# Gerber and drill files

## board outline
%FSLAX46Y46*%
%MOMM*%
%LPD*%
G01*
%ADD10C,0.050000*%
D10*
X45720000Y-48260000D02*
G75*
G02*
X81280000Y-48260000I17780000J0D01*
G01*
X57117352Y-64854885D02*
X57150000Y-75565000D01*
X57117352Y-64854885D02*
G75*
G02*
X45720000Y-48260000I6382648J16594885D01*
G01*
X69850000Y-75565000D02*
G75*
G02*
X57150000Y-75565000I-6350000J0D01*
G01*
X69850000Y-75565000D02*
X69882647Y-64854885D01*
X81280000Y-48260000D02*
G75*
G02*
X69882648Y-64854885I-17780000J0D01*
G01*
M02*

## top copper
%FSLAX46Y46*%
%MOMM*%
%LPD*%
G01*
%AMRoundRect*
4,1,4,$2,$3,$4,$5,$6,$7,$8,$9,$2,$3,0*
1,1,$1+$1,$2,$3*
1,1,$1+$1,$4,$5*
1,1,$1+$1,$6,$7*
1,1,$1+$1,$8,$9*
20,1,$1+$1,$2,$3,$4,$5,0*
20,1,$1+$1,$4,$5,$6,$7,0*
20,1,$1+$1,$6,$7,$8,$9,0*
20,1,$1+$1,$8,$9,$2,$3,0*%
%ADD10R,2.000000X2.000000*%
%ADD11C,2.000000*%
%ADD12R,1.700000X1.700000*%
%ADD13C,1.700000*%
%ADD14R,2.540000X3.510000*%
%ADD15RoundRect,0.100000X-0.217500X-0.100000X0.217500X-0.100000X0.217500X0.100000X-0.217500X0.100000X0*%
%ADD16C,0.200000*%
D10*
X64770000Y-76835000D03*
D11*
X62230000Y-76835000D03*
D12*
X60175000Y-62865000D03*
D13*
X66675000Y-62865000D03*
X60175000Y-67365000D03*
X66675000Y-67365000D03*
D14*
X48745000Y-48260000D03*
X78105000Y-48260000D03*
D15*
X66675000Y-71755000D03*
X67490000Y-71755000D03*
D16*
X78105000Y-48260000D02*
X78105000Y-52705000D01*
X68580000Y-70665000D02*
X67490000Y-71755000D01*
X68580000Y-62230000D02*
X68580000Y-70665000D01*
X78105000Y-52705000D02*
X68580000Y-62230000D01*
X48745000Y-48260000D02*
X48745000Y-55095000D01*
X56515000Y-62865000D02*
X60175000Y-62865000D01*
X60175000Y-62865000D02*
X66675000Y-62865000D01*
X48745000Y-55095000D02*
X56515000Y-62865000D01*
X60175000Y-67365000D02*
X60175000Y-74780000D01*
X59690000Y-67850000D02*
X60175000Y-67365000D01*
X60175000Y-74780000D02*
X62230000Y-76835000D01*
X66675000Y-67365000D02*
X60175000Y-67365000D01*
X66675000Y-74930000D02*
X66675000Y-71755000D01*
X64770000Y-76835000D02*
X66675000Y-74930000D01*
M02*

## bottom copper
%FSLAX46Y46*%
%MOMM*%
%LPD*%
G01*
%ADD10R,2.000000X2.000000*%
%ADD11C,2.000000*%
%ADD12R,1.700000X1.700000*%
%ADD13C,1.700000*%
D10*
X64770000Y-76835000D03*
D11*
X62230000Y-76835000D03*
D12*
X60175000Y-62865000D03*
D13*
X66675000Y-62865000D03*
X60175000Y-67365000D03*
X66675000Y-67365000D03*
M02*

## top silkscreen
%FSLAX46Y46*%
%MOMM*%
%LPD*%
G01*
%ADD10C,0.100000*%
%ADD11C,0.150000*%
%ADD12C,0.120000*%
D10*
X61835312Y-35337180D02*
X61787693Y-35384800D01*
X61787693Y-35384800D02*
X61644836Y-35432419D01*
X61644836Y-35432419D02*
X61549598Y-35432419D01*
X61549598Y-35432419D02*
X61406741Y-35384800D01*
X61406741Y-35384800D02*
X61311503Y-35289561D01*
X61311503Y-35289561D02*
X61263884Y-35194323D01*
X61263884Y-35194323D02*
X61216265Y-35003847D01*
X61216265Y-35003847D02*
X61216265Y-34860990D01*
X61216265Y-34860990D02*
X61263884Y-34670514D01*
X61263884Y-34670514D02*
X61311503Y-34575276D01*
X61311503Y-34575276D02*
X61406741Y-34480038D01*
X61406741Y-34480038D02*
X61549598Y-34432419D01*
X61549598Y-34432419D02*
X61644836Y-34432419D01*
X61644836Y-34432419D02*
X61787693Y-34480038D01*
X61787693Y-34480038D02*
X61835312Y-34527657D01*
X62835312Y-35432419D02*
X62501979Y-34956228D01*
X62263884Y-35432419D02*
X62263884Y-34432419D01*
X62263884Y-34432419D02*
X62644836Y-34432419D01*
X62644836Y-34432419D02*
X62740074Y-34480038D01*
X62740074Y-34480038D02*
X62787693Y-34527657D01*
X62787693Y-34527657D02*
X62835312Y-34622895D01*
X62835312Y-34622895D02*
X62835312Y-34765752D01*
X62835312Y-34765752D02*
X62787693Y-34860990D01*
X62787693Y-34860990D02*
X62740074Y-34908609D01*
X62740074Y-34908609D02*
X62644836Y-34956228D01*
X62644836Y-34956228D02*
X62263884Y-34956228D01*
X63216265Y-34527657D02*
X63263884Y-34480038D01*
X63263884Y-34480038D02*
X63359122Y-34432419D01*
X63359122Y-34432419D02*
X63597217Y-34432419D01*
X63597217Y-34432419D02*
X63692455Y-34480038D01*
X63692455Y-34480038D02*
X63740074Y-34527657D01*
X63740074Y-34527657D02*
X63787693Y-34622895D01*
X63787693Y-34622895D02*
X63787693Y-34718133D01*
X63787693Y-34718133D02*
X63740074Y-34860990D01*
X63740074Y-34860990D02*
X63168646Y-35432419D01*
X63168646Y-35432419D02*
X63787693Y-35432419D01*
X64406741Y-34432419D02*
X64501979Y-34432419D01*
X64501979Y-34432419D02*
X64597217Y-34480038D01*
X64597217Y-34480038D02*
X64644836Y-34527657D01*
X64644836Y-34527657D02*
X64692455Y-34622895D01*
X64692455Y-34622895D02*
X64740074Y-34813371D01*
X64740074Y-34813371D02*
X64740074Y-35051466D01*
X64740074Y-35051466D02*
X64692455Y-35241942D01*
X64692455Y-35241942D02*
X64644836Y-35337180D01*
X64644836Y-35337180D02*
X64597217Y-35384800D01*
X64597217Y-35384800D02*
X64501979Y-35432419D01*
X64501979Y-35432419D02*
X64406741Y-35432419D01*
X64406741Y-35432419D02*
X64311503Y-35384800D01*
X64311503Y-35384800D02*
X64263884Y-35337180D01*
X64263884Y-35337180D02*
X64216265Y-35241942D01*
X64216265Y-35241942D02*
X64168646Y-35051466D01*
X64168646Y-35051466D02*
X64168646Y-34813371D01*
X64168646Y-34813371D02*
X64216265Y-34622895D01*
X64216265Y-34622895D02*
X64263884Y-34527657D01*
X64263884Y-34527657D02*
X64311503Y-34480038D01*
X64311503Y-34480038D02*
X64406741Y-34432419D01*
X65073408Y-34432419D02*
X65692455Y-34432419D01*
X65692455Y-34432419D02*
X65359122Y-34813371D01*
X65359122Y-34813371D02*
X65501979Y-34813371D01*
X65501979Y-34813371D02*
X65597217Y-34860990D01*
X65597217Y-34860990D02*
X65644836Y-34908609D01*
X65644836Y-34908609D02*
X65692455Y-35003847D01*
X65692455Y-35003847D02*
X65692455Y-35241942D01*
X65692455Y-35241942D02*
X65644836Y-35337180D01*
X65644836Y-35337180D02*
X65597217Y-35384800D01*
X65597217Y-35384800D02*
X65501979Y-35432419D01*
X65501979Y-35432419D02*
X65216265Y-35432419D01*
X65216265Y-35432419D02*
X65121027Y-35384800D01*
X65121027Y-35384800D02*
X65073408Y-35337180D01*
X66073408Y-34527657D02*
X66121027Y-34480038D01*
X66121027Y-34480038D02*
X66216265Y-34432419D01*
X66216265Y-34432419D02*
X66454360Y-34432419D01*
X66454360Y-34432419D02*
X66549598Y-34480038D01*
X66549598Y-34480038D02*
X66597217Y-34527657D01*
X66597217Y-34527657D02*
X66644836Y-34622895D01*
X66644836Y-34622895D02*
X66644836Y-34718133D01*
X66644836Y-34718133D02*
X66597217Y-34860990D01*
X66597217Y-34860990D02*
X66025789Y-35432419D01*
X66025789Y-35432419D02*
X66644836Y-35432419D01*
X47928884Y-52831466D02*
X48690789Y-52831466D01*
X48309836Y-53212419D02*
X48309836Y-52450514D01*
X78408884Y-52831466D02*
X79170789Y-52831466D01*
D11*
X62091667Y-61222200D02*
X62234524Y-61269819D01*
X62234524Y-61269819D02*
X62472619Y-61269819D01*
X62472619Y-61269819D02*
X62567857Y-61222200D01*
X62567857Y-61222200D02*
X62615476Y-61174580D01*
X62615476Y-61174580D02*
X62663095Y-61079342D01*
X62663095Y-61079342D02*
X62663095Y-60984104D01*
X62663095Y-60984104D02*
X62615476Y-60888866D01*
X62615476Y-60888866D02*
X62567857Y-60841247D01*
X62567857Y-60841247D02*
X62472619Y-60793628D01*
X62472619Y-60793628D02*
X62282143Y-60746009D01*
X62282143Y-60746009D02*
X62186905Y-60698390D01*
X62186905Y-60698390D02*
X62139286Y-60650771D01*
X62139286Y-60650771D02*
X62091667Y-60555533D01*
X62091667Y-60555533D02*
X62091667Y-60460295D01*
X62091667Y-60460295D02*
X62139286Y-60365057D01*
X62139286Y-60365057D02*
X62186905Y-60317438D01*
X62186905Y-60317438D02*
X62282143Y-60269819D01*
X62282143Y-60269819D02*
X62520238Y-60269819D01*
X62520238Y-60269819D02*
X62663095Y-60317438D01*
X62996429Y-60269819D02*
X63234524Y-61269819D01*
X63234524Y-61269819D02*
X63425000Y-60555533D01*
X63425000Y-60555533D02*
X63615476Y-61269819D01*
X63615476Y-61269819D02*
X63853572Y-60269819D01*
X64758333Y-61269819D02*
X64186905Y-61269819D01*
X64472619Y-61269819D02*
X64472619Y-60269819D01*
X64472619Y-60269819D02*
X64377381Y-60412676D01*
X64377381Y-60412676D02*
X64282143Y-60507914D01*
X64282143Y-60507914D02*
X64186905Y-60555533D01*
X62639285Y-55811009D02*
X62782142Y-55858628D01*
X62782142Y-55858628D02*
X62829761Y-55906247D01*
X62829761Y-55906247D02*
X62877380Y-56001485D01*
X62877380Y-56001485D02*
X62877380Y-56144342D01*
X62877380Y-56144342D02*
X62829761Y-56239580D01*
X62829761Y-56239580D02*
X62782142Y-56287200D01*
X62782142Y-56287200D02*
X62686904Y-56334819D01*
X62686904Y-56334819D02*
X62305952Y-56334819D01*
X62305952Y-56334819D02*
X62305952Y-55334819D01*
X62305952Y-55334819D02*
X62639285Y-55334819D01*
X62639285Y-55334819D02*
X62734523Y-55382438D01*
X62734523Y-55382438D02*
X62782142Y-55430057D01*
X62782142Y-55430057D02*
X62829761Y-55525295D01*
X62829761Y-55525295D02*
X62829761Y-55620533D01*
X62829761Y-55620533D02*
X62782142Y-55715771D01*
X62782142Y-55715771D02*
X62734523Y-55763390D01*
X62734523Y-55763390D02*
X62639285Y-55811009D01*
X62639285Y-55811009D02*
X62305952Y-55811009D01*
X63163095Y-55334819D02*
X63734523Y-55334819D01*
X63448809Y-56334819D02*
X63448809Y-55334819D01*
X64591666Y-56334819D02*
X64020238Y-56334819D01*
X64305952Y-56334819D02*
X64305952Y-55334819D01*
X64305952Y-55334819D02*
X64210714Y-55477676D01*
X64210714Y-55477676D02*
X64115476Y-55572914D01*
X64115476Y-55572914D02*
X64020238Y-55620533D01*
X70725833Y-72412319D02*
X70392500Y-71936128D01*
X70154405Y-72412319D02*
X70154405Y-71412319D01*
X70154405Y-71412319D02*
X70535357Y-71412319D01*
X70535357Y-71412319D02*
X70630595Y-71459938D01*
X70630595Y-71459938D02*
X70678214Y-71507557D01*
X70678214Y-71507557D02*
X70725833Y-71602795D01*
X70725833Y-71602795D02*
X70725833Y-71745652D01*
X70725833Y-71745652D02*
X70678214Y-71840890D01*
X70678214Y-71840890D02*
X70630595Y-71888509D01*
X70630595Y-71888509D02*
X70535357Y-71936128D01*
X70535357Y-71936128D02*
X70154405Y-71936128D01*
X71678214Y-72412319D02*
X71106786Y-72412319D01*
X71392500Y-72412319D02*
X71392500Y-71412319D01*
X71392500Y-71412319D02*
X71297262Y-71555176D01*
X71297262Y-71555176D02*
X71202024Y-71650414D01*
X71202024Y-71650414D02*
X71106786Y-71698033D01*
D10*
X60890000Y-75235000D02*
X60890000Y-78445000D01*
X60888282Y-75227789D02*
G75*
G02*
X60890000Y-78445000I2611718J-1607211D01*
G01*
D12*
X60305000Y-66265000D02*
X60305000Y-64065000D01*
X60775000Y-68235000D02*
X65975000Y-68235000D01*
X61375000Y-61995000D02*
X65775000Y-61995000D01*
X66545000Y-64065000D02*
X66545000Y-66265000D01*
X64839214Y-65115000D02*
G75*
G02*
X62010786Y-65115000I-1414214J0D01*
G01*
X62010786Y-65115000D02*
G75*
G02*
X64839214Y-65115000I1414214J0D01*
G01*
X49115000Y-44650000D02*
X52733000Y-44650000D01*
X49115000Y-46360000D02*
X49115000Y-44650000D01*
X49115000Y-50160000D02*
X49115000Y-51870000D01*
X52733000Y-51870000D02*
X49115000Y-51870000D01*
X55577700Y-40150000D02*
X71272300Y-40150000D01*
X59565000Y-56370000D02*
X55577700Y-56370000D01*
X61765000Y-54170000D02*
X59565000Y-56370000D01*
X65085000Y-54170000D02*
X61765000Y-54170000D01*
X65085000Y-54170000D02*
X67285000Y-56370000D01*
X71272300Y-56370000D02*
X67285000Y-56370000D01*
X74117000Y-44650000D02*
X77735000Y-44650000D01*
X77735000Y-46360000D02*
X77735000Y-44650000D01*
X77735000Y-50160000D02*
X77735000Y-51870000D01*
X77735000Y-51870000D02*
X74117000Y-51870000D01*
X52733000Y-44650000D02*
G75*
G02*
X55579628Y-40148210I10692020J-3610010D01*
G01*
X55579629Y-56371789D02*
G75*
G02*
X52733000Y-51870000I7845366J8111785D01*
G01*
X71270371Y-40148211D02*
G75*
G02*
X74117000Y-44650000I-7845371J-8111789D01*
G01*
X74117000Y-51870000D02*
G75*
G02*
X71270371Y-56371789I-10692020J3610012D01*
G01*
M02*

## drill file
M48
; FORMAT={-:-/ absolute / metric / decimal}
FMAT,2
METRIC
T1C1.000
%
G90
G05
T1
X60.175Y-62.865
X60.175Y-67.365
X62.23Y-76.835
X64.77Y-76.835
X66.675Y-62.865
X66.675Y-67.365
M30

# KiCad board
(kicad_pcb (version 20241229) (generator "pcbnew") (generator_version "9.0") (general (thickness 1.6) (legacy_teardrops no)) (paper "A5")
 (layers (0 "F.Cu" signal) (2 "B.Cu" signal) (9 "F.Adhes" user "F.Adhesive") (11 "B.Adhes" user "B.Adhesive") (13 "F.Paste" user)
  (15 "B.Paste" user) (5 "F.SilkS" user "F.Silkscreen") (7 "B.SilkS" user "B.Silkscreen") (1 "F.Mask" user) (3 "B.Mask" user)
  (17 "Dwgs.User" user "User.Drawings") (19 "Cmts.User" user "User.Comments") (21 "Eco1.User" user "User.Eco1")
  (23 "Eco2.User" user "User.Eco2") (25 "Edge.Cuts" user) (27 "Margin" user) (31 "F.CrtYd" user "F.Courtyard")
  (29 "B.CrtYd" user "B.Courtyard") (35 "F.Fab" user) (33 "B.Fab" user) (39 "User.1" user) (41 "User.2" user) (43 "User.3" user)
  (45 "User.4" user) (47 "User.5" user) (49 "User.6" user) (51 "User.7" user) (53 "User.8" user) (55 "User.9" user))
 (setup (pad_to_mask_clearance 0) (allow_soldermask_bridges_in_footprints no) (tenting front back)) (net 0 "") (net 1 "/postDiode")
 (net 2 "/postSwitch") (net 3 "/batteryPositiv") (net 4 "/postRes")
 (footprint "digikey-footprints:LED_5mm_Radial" (layer "F.Cu") (at 62.23 76.835 180)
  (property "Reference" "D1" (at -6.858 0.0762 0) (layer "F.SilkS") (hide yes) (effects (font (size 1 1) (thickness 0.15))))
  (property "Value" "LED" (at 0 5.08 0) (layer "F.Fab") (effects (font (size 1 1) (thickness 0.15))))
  (fp_line (start 1.34 1.6) (end 1.34 -1.61) (stroke (width 0.1) (type solid)) (layer "F.SilkS"))
  (fp_arc (start 1.341718 1.607211) (mid -4.336626 0.001638) (end 1.34 -1.61) (stroke (width 0.1) (type solid)) (layer "F.SilkS"))
  (pad "1" thru_hole rect (at -2.54 0 180) (size 2 2) (drill 1) (layers "*.Cu" "*.Mask") (remove_unused_layers no) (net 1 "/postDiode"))
  (pad "2" thru_hole circle (at 0 0 180) (size 2 2) (drill 1) (layers "*.Cu" "*.Mask") (remove_unused_layers no) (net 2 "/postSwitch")))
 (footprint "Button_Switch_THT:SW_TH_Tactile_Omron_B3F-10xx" (layer "F.Cu") (at 60.175 62.865)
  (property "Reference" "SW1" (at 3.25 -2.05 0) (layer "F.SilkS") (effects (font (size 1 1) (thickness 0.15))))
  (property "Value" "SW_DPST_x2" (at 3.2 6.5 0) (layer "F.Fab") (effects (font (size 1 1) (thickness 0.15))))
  (fp_line (start 0.13 3.4) (end 0.13 1.2) (stroke (width 0.12) (type solid)) (layer "F.SilkS"))
  (fp_line (start 0.6 5.37) (end 5.8 5.37) (stroke (width 0.12) (type solid)) (layer "F.SilkS"))
  (fp_line (start 1.2 -0.87) (end 5.6 -0.87) (stroke (width 0.12) (type solid)) (layer "F.SilkS"))
  (fp_line (start 6.37 1.2) (end 6.37 3.4) (stroke (width 0.12) (type solid)) (layer "F.SilkS"))
  (fp_circle (center 3.25 2.25) (end 4.25 3.25) (stroke (width 0.12) (type solid)) (fill no) (layer "F.SilkS"))
  (pad "1" thru_hole rect (at 0 0) (size 1.7 1.7) (drill 1) (layers "*.Cu" "*.Mask") (remove_unused_layers no) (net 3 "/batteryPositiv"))
  (pad "1" thru_hole circle (at 6.5 0) (size 1.7 1.7) (drill 1) (layers "*.Cu" "*.Mask") (remove_unused_layers no) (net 3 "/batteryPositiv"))
  (pad "2" thru_hole circle (at 0 4.5) (size 1.7 1.7) (drill 1) (layers "*.Cu" "*.Mask") (remove_unused_layers no) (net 2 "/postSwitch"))
  (pad "2" thru_hole circle (at 6.5 4.5) (size 1.7 1.7) (drill 1) (layers "*.Cu" "*.Mask") (remove_unused_layers no) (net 2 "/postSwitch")))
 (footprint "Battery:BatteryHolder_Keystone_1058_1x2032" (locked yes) (layer "F.Cu") (at 63.425 48.26)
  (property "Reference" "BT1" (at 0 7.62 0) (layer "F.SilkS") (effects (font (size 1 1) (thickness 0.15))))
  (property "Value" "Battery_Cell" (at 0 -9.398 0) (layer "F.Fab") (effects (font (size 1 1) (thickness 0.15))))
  (fp_line (start -14.31 -3.61) (end -10.692 -3.61) (stroke (width 0.12) (type solid)) (layer "F.SilkS"))
  (fp_line (start -14.31 -1.9) (end -14.31 -3.61) (stroke (width 0.12) (type solid)) (layer "F.SilkS"))
  (fp_line (start -14.31 1.9) (end -14.31 3.61) (stroke (width 0.12) (type solid)) (layer "F.SilkS"))
  (fp_line (start -10.692 3.61) (end -14.31 3.61) (stroke (width 0.12) (type solid)) (layer "F.SilkS"))
  (fp_line (start -7.8473 -8.11) (end 7.8473 -8.11) (stroke (width 0.12) (type solid)) (layer "F.SilkS"))
  (fp_line (start -3.86 8.11) (end -7.8473 8.11) (stroke (width 0.12) (type solid)) (layer "F.SilkS"))
  (fp_line (start -1.66 5.91) (end -3.86 8.11) (stroke (width 0.12) (type solid)) (layer "F.SilkS"))
  (fp_line (start 1.66 5.91) (end -1.66 5.91) (stroke (width 0.12) (type solid)) (layer "F.SilkS"))
  (fp_line (start 1.66 5.91) (end 3.86 8.11) (stroke (width 0.12) (type solid)) (layer "F.SilkS"))
  (fp_line (start 7.8473 8.11) (end 3.86 8.11) (stroke (width 0.12) (type solid)) (layer "F.SilkS"))
  (fp_line (start 10.692 -3.61) (end 14.31 -3.61) (stroke (width 0.12) (type solid)) (layer "F.SilkS"))
  (fp_line (start 14.31 -1.9) (end 14.31 -3.61) (stroke (width 0.12) (type solid)) (layer "F.SilkS"))
  (fp_line (start 14.31 1.9) (end 14.31 3.61) (stroke (width 0.12) (type solid)) (layer "F.SilkS"))
  (fp_line (start 14.31 3.61) (end 10.692 3.61) (stroke (width 0.12) (type solid)) (layer "F.SilkS"))
  (fp_arc (start -10.692 -3.61) (mid -9.538084 -6.031244) (end -7.845371 -8.111789) (stroke (width 0.12) (type solid)) (layer "F.SilkS"))
  (fp_arc (start -7.845371 8.111789) (mid -9.538085 6.031244) (end -10.692 3.61) (stroke (width 0.12) (type solid)) (layer "F.SilkS"))
  (fp_arc (start 7.845371 -8.111789) (mid 9.538085 -6.031244) (end 10.692 -3.61) (stroke (width 0.12) (type solid)) (layer "F.SilkS"))
  (fp_arc (start 10.692 3.61) (mid 9.538084 6.031244) (end 7.845371 8.111789) (stroke (width 0.12) (type solid)) (layer "F.SilkS"))
  (pad "1" smd rect (at -14.68 0) (size 2.54 3.51) (layers "F.Cu" "F.Mask" "F.Paste") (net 3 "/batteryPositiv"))
  (pad "2" smd rect (at 14.68 0) (size 2.54 3.51) (layers "F.Cu" "F.Mask" "F.Paste") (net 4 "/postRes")))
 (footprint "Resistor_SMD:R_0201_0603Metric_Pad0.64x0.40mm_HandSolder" (layer "F.Cu") (at 67.0825 71.755)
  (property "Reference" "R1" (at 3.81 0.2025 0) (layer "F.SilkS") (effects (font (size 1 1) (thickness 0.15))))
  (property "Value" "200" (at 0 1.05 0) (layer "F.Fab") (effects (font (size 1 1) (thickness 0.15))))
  (pad "" smd roundrect (at -0.4325 0) (size 0.458 0.36) (layers "F.Paste") (roundrect_rratio 0.25))
  (pad "" smd roundrect (at 0.4325 0) (size 0.458 0.36) (layers "F.Paste") (roundrect_rratio 0.25))
  (pad "1" smd roundrect (at -0.4075 0) (size 0.635 0.4) (layers "F.Cu" "F.Mask") (roundrect_rratio 0.25) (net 1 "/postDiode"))
  (pad "2" smd roundrect (at 0.4075 0) (size 0.635 0.4) (layers "F.Cu" "F.Mask") (roundrect_rratio 0.25) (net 4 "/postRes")))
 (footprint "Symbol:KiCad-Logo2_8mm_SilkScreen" (layer "B.Cu") (at 62.865 47.625 180)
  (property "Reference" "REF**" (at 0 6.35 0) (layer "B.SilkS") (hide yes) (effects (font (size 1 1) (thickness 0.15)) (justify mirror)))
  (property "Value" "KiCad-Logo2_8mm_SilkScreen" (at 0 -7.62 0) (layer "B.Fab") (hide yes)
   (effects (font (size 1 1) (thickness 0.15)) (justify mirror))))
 (gr_arc (start 45.72 48.26) (mid 63.5 30.48) (end 81.28 48.26) (stroke (width 0.05) (type default)) (layer "Edge.Cuts"))
 (gr_line (start 57.117352 64.854885) (end 57.15 75.565) (stroke (width 0.05) (type default)) (layer "Edge.Cuts"))
 (gr_arc (start 57.117352 64.854885) (mid 48.84374 58.325906) (end 45.72 48.26) (stroke (width 0.05) (type default)) (layer "Edge.Cuts"))
 (gr_arc (start 69.85 75.565) (mid 63.5 81.915) (end 57.15 75.565) (stroke (width 0.05) (type default)) (layer "Edge.Cuts"))
 (gr_line (start 69.85 75.565) (end 69.882647 64.854885) (stroke (width 0.05) (type default)) (layer "Edge.Cuts"))
 (gr_arc (start 81.28 48.26) (mid 78.156259 58.325906) (end 69.882648 64.854885) (stroke (width 0.05) (type default)) (layer "Edge.Cuts"))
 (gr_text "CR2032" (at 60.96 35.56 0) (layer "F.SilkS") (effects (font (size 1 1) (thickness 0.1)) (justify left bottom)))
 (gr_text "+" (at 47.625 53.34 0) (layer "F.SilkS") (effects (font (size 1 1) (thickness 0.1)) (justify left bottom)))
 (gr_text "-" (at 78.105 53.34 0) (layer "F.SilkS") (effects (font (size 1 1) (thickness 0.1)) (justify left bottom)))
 (segment (start 78.105 48.26) (end 78.105 52.705) (width 0.2) (layer "F.Cu") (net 4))
 (segment (start 68.58 70.665) (end 67.49 71.755) (width 0.2) (layer "F.Cu") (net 4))
 (segment (start 68.58 62.23) (end 68.58 70.665) (width 0.2) (layer "F.Cu") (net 4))
 (segment (start 78.105 52.705) (end 68.58 62.23) (width 0.2) (layer "F.Cu") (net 4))
 (segment (start 48.745 48.26) (end 48.745 55.095) (width 0.2) (layer "F.Cu") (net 3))
 (segment (start 56.515 62.865) (end 60.175 62.865) (width 0.2) (layer "F.Cu") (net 3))
 (segment (start 60.175 62.865) (end 66.675 62.865) (width 0.2) (layer "F.Cu") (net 3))
 (segment (start 48.745 55.095) (end 56.515 62.865) (width 0.2) (layer "F.Cu") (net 3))
 (segment (start 60.175 67.365) (end 60.175 74.78) (width 0.2) (layer "F.Cu") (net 2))
 (segment (start 59.69 67.85) (end 60.175 67.365) (width 0.2) (layer "F.Cu") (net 2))
 (segment (start 60.175 74.78) (end 62.23 76.835) (width 0.2) (layer "F.Cu") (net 2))
 (segment (start 66.675 67.365) (end 60.175 67.365) (width 0.2) (layer "F.Cu") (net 2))
 (segment (start 66.675 74.93) (end 66.675 71.755) (width 0.2) (layer "F.Cu") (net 1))
 (segment (start 64.77 76.835) (end 66.675 74.93) (width 0.2) (layer "F.Cu") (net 1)))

